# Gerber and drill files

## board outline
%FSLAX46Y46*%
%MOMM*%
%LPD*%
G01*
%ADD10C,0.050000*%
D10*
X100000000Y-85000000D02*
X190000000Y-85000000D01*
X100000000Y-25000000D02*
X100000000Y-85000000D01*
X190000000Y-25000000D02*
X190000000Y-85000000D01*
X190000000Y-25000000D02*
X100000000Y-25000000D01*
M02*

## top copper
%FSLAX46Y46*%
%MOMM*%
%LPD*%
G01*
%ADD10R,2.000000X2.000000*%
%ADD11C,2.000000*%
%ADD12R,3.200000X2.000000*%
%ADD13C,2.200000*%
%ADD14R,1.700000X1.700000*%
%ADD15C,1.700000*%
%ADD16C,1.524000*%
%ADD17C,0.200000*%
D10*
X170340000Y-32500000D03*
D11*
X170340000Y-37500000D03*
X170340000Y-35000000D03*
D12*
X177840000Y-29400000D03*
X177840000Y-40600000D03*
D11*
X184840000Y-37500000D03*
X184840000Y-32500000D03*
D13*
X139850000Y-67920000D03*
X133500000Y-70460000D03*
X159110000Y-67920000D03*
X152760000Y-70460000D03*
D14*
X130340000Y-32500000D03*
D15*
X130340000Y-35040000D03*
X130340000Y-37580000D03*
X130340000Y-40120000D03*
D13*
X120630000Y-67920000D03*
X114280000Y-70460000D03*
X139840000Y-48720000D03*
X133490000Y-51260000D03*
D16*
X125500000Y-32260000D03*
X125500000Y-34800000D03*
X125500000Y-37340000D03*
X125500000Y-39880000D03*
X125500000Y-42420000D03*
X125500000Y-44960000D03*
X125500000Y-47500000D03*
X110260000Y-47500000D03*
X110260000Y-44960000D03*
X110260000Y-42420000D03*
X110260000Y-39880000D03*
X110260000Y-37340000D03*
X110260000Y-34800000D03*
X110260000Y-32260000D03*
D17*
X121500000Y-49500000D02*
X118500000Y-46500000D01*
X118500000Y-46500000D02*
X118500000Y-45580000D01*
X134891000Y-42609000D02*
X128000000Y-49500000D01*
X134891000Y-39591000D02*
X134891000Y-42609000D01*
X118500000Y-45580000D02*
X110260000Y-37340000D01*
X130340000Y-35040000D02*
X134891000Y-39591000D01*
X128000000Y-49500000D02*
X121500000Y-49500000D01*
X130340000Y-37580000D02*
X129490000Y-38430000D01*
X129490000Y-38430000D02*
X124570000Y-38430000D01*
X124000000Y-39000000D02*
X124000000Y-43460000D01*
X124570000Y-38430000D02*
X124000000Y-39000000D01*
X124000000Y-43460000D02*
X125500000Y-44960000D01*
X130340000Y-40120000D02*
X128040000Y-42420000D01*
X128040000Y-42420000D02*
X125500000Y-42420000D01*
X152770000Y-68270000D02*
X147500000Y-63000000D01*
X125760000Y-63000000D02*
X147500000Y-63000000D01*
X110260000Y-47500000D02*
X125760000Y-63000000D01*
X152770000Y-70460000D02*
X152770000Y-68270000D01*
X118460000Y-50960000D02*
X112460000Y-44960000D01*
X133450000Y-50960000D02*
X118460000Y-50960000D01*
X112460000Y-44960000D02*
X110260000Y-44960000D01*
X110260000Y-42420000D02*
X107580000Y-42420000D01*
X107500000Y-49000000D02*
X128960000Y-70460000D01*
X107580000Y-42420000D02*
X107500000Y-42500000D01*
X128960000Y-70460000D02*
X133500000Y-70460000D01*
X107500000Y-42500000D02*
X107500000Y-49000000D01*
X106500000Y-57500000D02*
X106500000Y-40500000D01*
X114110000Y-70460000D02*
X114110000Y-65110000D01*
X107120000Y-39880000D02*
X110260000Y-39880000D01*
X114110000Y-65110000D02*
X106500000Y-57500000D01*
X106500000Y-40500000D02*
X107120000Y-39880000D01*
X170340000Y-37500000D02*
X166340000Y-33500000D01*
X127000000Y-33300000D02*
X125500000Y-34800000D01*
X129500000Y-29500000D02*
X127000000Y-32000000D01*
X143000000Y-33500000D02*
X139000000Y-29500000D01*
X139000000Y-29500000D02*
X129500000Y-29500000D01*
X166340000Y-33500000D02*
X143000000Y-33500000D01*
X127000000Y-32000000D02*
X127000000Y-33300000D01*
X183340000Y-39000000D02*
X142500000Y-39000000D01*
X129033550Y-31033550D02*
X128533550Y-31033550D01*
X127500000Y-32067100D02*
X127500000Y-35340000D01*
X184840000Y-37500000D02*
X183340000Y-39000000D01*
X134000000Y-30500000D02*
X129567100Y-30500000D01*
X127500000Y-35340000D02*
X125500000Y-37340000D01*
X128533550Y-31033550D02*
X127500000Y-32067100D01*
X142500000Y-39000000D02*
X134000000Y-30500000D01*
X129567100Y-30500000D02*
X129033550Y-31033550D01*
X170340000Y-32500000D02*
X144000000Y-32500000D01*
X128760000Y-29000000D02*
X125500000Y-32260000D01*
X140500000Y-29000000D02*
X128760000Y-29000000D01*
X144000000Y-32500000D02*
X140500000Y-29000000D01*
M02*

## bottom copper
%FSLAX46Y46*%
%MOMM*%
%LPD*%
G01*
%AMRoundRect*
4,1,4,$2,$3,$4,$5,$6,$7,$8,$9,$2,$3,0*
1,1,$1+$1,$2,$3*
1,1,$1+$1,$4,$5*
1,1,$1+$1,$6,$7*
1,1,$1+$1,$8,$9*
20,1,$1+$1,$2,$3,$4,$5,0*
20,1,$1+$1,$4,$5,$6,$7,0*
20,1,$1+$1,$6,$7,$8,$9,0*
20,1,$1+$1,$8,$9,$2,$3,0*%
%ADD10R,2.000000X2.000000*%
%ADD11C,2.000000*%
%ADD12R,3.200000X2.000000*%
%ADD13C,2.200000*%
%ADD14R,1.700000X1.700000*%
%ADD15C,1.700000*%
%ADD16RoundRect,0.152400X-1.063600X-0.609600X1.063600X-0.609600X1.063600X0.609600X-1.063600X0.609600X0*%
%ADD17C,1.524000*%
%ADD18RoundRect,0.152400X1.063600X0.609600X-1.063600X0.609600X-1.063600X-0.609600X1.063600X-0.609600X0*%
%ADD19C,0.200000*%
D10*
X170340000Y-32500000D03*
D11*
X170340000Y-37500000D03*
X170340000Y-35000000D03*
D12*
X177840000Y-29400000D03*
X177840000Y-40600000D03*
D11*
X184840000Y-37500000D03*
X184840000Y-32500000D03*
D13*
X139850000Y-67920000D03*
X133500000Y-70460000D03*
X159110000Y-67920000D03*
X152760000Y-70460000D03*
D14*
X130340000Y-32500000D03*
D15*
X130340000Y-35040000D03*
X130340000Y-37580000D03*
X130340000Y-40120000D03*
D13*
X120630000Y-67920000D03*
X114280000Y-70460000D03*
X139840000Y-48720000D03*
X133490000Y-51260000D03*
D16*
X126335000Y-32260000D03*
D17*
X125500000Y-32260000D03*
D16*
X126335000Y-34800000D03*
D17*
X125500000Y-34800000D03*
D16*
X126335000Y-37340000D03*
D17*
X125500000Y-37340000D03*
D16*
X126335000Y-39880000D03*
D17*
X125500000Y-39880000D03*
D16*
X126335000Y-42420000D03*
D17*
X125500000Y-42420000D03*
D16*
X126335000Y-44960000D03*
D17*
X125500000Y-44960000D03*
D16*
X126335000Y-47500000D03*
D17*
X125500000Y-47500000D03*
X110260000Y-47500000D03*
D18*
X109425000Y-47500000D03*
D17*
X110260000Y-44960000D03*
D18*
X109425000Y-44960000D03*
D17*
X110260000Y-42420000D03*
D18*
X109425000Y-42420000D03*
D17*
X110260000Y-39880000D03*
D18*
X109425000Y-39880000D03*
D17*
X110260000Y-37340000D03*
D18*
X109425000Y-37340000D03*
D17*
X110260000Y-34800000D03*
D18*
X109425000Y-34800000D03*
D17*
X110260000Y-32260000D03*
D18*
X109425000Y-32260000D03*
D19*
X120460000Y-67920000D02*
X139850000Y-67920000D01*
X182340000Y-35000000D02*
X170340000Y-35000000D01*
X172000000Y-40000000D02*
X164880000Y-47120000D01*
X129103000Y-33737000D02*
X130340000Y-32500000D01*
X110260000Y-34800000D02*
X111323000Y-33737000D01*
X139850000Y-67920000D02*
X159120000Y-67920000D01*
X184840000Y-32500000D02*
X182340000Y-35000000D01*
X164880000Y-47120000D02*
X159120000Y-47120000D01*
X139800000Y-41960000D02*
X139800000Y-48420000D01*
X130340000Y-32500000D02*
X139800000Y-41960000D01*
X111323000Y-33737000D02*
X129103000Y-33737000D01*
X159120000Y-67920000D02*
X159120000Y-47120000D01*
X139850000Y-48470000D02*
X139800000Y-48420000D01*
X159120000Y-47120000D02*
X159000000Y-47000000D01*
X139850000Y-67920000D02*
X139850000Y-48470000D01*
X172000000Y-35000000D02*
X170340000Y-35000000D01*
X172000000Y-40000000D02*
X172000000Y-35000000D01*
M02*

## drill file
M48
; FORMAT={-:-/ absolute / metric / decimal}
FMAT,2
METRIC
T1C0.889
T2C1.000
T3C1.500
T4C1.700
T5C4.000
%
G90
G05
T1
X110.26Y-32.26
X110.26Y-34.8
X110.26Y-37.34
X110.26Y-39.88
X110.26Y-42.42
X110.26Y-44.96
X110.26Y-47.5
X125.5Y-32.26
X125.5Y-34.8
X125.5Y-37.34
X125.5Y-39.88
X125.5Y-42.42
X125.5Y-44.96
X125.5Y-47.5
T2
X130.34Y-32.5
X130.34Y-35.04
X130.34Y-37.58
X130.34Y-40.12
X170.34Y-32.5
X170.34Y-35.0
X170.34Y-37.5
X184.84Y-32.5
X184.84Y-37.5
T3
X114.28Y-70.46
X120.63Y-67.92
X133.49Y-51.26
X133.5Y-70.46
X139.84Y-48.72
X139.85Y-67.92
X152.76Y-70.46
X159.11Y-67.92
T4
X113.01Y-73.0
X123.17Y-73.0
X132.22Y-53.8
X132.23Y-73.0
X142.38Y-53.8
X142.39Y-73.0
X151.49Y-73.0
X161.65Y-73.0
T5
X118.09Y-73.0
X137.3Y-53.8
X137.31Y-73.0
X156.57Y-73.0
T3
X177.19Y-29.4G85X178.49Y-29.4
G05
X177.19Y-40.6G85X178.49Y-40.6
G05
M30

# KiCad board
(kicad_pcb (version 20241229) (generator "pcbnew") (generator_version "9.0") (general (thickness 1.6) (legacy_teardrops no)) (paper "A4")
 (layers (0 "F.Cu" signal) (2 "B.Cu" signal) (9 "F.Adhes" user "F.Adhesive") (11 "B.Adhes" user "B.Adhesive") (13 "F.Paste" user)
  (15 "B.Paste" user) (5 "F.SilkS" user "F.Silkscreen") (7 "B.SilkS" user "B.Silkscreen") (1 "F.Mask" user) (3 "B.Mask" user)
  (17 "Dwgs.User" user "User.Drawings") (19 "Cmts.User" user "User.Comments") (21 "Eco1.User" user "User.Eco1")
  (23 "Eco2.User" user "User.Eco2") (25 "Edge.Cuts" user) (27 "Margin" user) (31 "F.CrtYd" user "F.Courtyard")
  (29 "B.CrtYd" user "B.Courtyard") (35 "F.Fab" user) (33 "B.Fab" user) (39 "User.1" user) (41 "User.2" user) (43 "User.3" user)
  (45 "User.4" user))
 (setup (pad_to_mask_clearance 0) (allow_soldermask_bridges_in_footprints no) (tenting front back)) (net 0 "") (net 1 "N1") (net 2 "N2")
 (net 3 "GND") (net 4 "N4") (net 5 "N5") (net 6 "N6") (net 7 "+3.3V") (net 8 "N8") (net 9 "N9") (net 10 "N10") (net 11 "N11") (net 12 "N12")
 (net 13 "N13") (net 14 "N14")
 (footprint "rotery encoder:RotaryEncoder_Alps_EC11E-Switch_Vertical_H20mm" (layer "F.Cu") (at 170.34 32.5)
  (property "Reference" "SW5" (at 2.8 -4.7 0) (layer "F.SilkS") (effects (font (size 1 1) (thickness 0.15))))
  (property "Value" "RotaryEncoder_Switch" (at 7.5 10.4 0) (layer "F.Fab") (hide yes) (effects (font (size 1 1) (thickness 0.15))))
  (pad "A" thru_hole rect (at 0 0) (size 2 2) (drill 1) (layers "*.Cu" "*.Mask") (remove_unused_layers no) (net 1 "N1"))
  (pad "B" thru_hole circle (at 0 5) (size 2 2) (drill 1) (layers "*.Cu" "*.Mask") (remove_unused_layers no) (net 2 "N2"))
  (pad "C" thru_hole circle (at 0 2.5) (size 2 2) (drill 1) (layers "*.Cu" "*.Mask") (remove_unused_layers no) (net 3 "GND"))
  (pad "MP" thru_hole rect (at 7.5 -3.1) (size 3.2 2) (drill oval 2.8 1.5) (layers "*.Cu" "*.Mask") (remove_unused_layers no))
  (pad "MP" thru_hole rect (at 7.5 8.1) (size 3.2 2) (drill oval 2.8 1.5) (layers "*.Cu" "*.Mask") (remove_unused_layers no))
  (pad "S1" thru_hole circle (at 14.5 5) (size 2 2) (drill 1) (layers "*.Cu" "*.Mask") (remove_unused_layers no) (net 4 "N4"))
  (pad "S2" thru_hole circle (at 14.5 0) (size 2 2) (drill 1) (layers "*.Cu" "*.Mask") (remove_unused_layers no) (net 3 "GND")))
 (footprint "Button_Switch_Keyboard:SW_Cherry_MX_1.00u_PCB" (layer "F.Cu") (at 139.85 67.92)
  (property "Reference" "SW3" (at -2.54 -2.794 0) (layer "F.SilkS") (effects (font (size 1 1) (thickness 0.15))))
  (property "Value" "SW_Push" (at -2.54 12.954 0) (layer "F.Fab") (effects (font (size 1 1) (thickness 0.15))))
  (pad "" np_thru_hole circle (at -7.62 5.08) (size 1.7 1.7) (drill 1.7) (layers "*.Cu" "*.Mask"))
  (pad "" np_thru_hole circle (at -2.54 5.08) (size 4 4) (drill 4) (layers "*.Cu" "*.Mask"))
  (pad "" np_thru_hole circle (at 2.54 5.08) (size 1.7 1.7) (drill 1.7) (layers "*.Cu" "*.Mask"))
  (pad "1" thru_hole circle (at 0 0) (size 2.2 2.2) (drill 1.5) (layers "*.Cu" "*.Mask") (remove_unused_layers no) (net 3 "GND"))
  (pad "2" thru_hole circle (at -6.35 2.54) (size 2.2 2.2) (drill 1.5) (layers "*.Cu" "*.Mask") (remove_unused_layers no) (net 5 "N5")))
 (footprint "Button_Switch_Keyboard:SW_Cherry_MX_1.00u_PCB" (layer "F.Cu") (at 159.11 67.92)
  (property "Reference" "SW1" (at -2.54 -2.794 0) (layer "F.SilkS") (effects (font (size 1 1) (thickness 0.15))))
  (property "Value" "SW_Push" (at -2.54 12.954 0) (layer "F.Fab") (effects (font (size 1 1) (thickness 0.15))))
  (pad "" np_thru_hole circle (at -7.62 5.08) (size 1.7 1.7) (drill 1.7) (layers "*.Cu" "*.Mask"))
  (pad "" np_thru_hole circle (at -2.54 5.08) (size 4 4) (drill 4) (layers "*.Cu" "*.Mask"))
  (pad "" np_thru_hole circle (at 2.54 5.08) (size 1.7 1.7) (drill 1.7) (layers "*.Cu" "*.Mask"))
  (pad "1" thru_hole circle (at 0 0) (size 2.2 2.2) (drill 1.5) (layers "*.Cu" "*.Mask") (remove_unused_layers no) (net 3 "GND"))
  (pad "2" thru_hole circle (at -6.35 2.54) (size 2.2 2.2) (drill 1.5) (layers "*.Cu" "*.Mask") (remove_unused_layers no) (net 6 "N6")))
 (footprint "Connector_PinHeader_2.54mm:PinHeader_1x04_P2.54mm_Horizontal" (layer "F.Cu") (at 130.34 32.5)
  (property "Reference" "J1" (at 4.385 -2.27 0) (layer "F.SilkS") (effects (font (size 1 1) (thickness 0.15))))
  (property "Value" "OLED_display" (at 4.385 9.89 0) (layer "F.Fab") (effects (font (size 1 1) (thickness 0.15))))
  (pad "1" thru_hole rect (at 0 0) (size 1.7 1.7) (drill 1) (layers "*.Cu" "*.Mask") (remove_unused_layers no) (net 3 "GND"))
  (pad "2" thru_hole circle (at 0 2.54) (size 1.7 1.7) (drill 1) (layers "*.Cu" "*.Mask") (remove_unused_layers no) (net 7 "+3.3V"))
  (pad "3" thru_hole circle (at 0 5.08) (size 1.7 1.7) (drill 1) (layers "*.Cu" "*.Mask") (remove_unused_layers no) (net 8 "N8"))
  (pad "4" thru_hole circle (at 0 7.62) (size 1.7 1.7) (drill 1) (layers "*.Cu" "*.Mask") (remove_unused_layers no) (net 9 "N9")))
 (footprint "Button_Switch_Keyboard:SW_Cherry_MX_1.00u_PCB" (layer "F.Cu") (at 120.63 67.92)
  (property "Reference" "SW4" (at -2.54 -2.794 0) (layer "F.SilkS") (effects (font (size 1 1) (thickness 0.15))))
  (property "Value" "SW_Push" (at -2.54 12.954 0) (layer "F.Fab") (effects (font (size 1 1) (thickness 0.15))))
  (pad "" np_thru_hole circle (at -7.62 5.08) (size 1.7 1.7) (drill 1.7) (layers "*.Cu" "*.Mask"))
  (pad "" np_thru_hole circle (at -2.54 5.08) (size 4 4) (drill 4) (layers "*.Cu" "*.Mask"))
  (pad "" np_thru_hole circle (at 2.54 5.08) (size 1.7 1.7) (drill 1.7) (layers "*.Cu" "*.Mask"))
  (pad "1" thru_hole circle (at 0 0) (size 2.2 2.2) (drill 1.5) (layers "*.Cu" "*.Mask") (remove_unused_layers no) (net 3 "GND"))
  (pad "2" thru_hole circle (at -6.35 2.54) (size 2.2 2.2) (drill 1.5) (layers "*.Cu" "*.Mask") (remove_unused_layers no) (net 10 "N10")))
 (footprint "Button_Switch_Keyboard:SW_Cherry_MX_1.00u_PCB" (layer "F.Cu") (at 139.84 48.72)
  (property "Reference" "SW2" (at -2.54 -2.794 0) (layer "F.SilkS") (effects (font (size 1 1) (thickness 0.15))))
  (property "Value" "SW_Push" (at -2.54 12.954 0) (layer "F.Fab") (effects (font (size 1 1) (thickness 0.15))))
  (pad "" np_thru_hole circle (at -7.62 5.08) (size 1.7 1.7) (drill 1.7) (layers "*.Cu" "*.Mask"))
  (pad "" np_thru_hole circle (at -2.54 5.08) (size 4 4) (drill 4) (layers "*.Cu" "*.Mask"))
  (pad "" np_thru_hole circle (at 2.54 5.08) (size 1.7 1.7) (drill 1.7) (layers "*.Cu" "*.Mask"))
  (pad "1" thru_hole circle (at 0 0) (size 2.2 2.2) (drill 1.5) (layers "*.Cu" "*.Mask") (remove_unused_layers no) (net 3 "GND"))
  (pad "2" thru_hole circle (at -6.35 2.54) (size 2.2 2.2) (drill 1.5) (layers "*.Cu" "*.Mask") (remove_unused_layers no) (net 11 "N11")))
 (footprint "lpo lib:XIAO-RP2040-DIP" (layer "B.Cu") (at 117.88 39.88 180)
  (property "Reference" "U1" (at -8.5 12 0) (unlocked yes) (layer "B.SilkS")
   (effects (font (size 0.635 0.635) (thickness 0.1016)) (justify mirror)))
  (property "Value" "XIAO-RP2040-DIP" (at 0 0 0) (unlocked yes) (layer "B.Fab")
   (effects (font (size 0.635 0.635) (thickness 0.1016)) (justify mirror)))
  (pad "1" smd roundrect (at -8.455 7.62) (size 2.432 1.524) (layers "B.Cu" "B.Mask") (roundrect_rratio 0.1) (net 1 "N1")
   (thermal_bridge_angle 45))
  (pad "1" thru_hole circle (at -7.62 7.62) (size 1.524 1.524) (drill 0.889) (layers "*.Cu" "*.Mask") (remove_unused_layers no) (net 1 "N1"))
  (pad "2" smd roundrect (at -8.455 5.08) (size 2.432 1.524) (layers "B.Cu" "B.Mask") (roundrect_rratio 0.1) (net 2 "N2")
   (thermal_bridge_angle 45))
  (pad "2" thru_hole circle (at -7.62 5.08) (size 1.524 1.524) (drill 0.889) (layers "*.Cu" "*.Mask") (remove_unused_layers no) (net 2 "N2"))
  (pad "3" smd roundrect (at -8.455 2.54) (size 2.432 1.524) (layers "B.Cu" "B.Mask") (roundrect_rratio 0.1) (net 4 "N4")
   (thermal_bridge_angle 45))
  (pad "3" thru_hole circle (at -7.62 2.54) (size 1.524 1.524) (drill 0.889) (layers "*.Cu" "*.Mask") (remove_unused_layers no) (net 4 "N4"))
  (pad "4" smd roundrect (at -8.455 0) (size 2.432 1.524) (layers "B.Cu" "B.Mask") (roundrect_rratio 0.1) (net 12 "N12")
   (thermal_bridge_angle 45))
  (pad "4" thru_hole circle (at -7.62 0) (size 1.524 1.524) (drill 0.889) (layers "*.Cu" "*.Mask") (remove_unused_layers no) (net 12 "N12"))
  (pad "5" smd roundrect (at -8.455 -2.54) (size 2.432 1.524) (layers "B.Cu" "B.Mask") (roundrect_rratio 0.1) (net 9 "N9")
   (thermal_bridge_angle 45))
  (pad "5" thru_hole circle (at -7.62 -2.54) (size 1.524 1.524) (drill 0.889) (layers "*.Cu" "*.Mask") (remove_unused_layers no)
   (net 9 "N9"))
  (pad "6" smd roundrect (at -8.455 -5.08) (size 2.432 1.524) (layers "B.Cu" "B.Mask") (roundrect_rratio 0.1) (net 8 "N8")
   (thermal_bridge_angle 45))
  (pad "6" thru_hole circle (at -7.62 -5.08) (size 1.524 1.524) (drill 0.889) (layers "*.Cu" "*.Mask") (remove_unused_layers no)
   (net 8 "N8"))
  (pad "7" smd roundrect (at -8.455 -7.62) (size 2.432 1.524) (layers "B.Cu" "B.Mask") (roundrect_rratio 0.1) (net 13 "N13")
   (thermal_bridge_angle 45))
  (pad "7" thru_hole circle (at -7.62 -7.62) (size 1.524 1.524) (drill 0.889) (layers "*.Cu" "*.Mask") (remove_unused_layers no)
   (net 13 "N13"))
  (pad "8" thru_hole circle (at 7.62 -7.62 180) (size 1.524 1.524) (drill 0.889) (layers "*.Cu" "*.Mask") (remove_unused_layers no)
   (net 6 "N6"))
  (pad "8" smd roundrect (at 8.455 -7.62 180) (size 2.432 1.524) (layers "B.Cu" "B.Mask") (roundrect_rratio 0.1) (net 6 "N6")
   (thermal_bridge_angle 45))
  (pad "9" thru_hole circle (at 7.62 -5.08 180) (size 1.524 1.524) (drill 0.889) (layers "*.Cu" "*.Mask") (remove_unused_layers no)
   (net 11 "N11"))
  (pad "9" smd roundrect (at 8.455 -5.08 180) (size 2.432 1.524) (layers "B.Cu" "B.Mask") (roundrect_rratio 0.1) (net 11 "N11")
   (thermal_bridge_angle 45))
  (pad "10" thru_hole circle (at 7.62 -2.54 180) (size 1.524 1.524) (drill 0.889) (layers "*.Cu" "*.Mask") (remove_unused_layers no)
   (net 5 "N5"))
  (pad "10" smd roundrect (at 8.455 -2.54 180) (size 2.432 1.524) (layers "B.Cu" "B.Mask") (roundrect_rratio 0.1) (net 5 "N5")
   (thermal_bridge_angle 45))
  (pad "11" thru_hole circle (at 7.62 0 180) (size 1.524 1.524) (drill 0.889) (layers "*.Cu" "*.Mask") (remove_unused_layers no)
   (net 10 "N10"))
  (pad "11" smd roundrect (at 8.455 0 180) (size 2.432 1.524) (layers "B.Cu" "B.Mask") (roundrect_rratio 0.1) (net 10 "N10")
   (thermal_bridge_angle 45))
  (pad "12" thru_hole circle (at 7.62 2.54 180) (size 1.524 1.524) (drill 0.889) (layers "*.Cu" "*.Mask") (remove_unused_layers no)
   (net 7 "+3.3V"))
  (pad "12" smd roundrect (at 8.455 2.54 180) (size 2.432 1.524) (layers "B.Cu" "B.Mask") (roundrect_rratio 0.1) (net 7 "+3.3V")
   (thermal_bridge_angle 45))
  (pad "13" thru_hole circle (at 7.62 5.08 180) (size 1.524 1.524) (drill 0.889) (layers "*.Cu" "*.Mask") (remove_unused_layers no)
   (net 3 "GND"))
  (pad "13" smd roundrect (at 8.455 5.08 180) (size 2.432 1.524) (layers "B.Cu" "B.Mask") (roundrect_rratio 0.1) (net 3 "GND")
   (thermal_bridge_angle 45))
  (pad "14" thru_hole circle (at 7.62 7.62 180) (size 1.524 1.524) (drill 0.889) (layers "*.Cu" "*.Mask") (remove_unused_layers no)
   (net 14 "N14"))
  (pad "14" smd roundrect (at 8.455 7.62 180) (size 2.432 1.524) (layers "B.Cu" "B.Mask") (roundrect_rratio 0.1) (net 14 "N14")
   (thermal_bridge_angle 45)))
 (gr_line (start 100 85) (end 190 85) (stroke (width 0.05) (type default)) (layer "Edge.Cuts"))
 (gr_line (start 100 25) (end 100 85) (stroke (width 0.05) (type default)) (layer "Edge.Cuts"))
 (gr_line (start 190 25) (end 190 85) (stroke (width 0.05) (type default)) (layer "Edge.Cuts"))
 (gr_line (start 190 25) (end 100 25) (stroke (width 0.05) (type default)) (layer "Edge.Cuts"))
 (segment (start 121.5 49.5) (end 118.5 46.5) (width 0.2) (layer "F.Cu") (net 7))
 (segment (start 118.5 46.5) (end 118.5 45.58) (width 0.2) (layer "F.Cu") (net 7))
 (segment (start 134.891 42.609) (end 128 49.5) (width 0.2) (layer "F.Cu") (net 7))
 (segment (start 134.891 39.591) (end 134.891 42.609) (width 0.2) (layer "F.Cu") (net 7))
 (segment (start 118.5 45.58) (end 110.26 37.34) (width 0.2) (layer "F.Cu") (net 7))
 (segment (start 130.34 35.04) (end 134.891 39.591) (width 0.2) (layer "F.Cu") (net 7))
 (segment (start 128 49.5) (end 121.5 49.5) (width 0.2) (layer "F.Cu") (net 7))
 (segment (start 120.46 67.92) (end 139.85 67.92) (width 0.2) (layer "B.Cu") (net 3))
 (segment (start 182.34 35) (end 170.34 35) (width 0.2) (layer "B.Cu") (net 3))
 (segment (start 172 40) (end 164.88 47.12) (width 0.2) (layer "B.Cu") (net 3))
 (segment (start 129.103 33.737) (end 130.34 32.5) (width 0.2) (layer "B.Cu") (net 3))
 (segment (start 110.26 34.8) (end 111.323 33.737) (width 0.2) (layer "B.Cu") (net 3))
 (segment (start 139.85 67.92) (end 159.12 67.92) (width 0.2) (layer "B.Cu") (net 3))
 (segment (start 184.84 32.5) (end 182.34 35) (width 0.2) (layer "B.Cu") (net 3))
 (segment (start 164.88 47.12) (end 159.12 47.12) (width 0.2) (layer "B.Cu") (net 3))
 (segment (start 139.8 41.96) (end 139.8 48.42) (width 0.2) (layer "B.Cu") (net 3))
 (segment (start 130.34 32.5) (end 139.8 41.96) (width 0.2) (layer "B.Cu") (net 3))
 (segment (start 111.323 33.737) (end 129.103 33.737) (width 0.2) (layer "B.Cu") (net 3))
 (segment (start 159.12 67.92) (end 159.12 47.12) (width 0.2) (layer "B.Cu") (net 3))
 (segment (start 139.85 48.47) (end 139.8 48.42) (width 0.2) (layer "B.Cu") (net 3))
 (segment (start 159.12 47.12) (end 159 47) (width 0.2) (layer "B.Cu") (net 3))
 (segment (start 139.85 67.92) (end 139.85 48.47) (width 0.2) (layer "B.Cu") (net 3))
 (segment (start 172 35) (end 170.34 35) (width 0.2) (layer "B.Cu") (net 3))
 (segment (start 172 40) (end 172 35) (width 0.2) (layer "B.Cu") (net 3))
 (segment (start 130.34 37.58) (end 129.49 38.43) (width 0.2) (layer "F.Cu") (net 8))
 (segment (start 129.49 38.43) (end 124.57 38.43) (width 0.2) (layer "F.Cu") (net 8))
 (segment (start 124 39) (end 124 43.46) (width 0.2) (layer "F.Cu") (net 8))
 (segment (start 124.57 38.43) (end 124 39) (width 0.2) (layer "F.Cu") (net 8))
 (segment (start 124 43.46) (end 125.5 44.96) (width 0.2) (layer "F.Cu") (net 8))
 (segment (start 130.34 40.12) (end 128.04 42.42) (width 0.2) (layer "F.Cu") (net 9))
 (segment (start 128.04 42.42) (end 125.5 42.42) (width 0.2) (layer "F.Cu") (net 9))
 (segment (start 152.77 68.27) (end 147.5 63) (width 0.2) (layer "F.Cu") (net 6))
 (segment (start 125.76 63) (end 147.5 63) (width 0.2) (layer "F.Cu") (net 6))
 (segment (start 110.26 47.5) (end 125.76 63) (width 0.2) (layer "F.Cu") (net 6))
 (segment (start 152.77 70.46) (end 152.77 68.27) (width 0.2) (layer "F.Cu") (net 6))
 (segment (start 118.46 50.96) (end 112.46 44.96) (width 0.2) (layer "F.Cu") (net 11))
 (segment (start 133.45 50.96) (end 118.46 50.96) (width 0.2) (layer "F.Cu") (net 11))
 (segment (start 112.46 44.96) (end 110.26 44.96) (width 0.2) (layer "F.Cu") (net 11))
 (segment (start 110.26 42.42) (end 107.58 42.42) (width 0.2) (layer "F.Cu") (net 5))
 (segment (start 107.5 49) (end 128.96 70.46) (width 0.2) (layer "F.Cu") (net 5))
 (segment (start 107.58 42.42) (end 107.5 42.5) (width 0.2) (layer "F.Cu") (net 5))
 (segment (start 128.96 70.46) (end 133.5 70.46) (width 0.2) (layer "F.Cu") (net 5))
 (segment (start 107.5 42.5) (end 107.5 49) (width 0.2) (layer "F.Cu") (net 5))
 (segment (start 106.5 57.5) (end 106.5 40.5) (width 0.2) (layer "F.Cu") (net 10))
 (segment (start 114.11 70.46) (end 114.11 65.11) (width 0.2) (layer "F.Cu") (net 10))
 (segment (start 107.12 39.88) (end 110.26 39.88) (width 0.2) (layer "F.Cu") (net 10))
 (segment (start 114.11 65.11) (end 106.5 57.5) (width 0.2) (layer "F.Cu") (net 10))
 (segment (start 106.5 40.5) (end 107.12 39.88) (width 0.2) (layer "F.Cu") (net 10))
 (segment (start 170.34 37.5) (end 166.34 33.5) (width 0.2) (layer "F.Cu") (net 2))
 (segment (start 127 33.3) (end 125.5 34.8) (width 0.2) (layer "F.Cu") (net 2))
 (segment (start 129.5 29.5) (end 127 32) (width 0.2) (layer "F.Cu") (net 2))
 (segment (start 143 33.5) (end 139 29.5) (width 0.2) (layer "F.Cu") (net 2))
 (segment (start 139 29.5) (end 129.5 29.5) (width 0.2) (layer "F.Cu") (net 2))
 (segment (start 166.34 33.5) (end 143 33.5) (width 0.2) (layer "F.Cu") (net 2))
 (segment (start 127 32) (end 127 33.3) (width 0.2) (layer "F.Cu") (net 2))
 (segment (start 183.34 39) (end 142.5 39) (width 0.2) (layer "F.Cu") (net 4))
 (segment (start 129.03355 31.03355) (end 128.53355 31.03355) (width 0.2) (layer "F.Cu") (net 4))
 (segment (start 127.5 32.0671) (end 127.5 35.34) (width 0.2) (layer "F.Cu") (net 4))
 (segment (start 184.84 37.5) (end 183.34 39) (width 0.2) (layer "F.Cu") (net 4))
 (segment (start 134 30.5) (end 129.5671 30.5) (width 0.2) (layer "F.Cu") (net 4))
 (segment (start 127.5 35.34) (end 125.5 37.34) (width 0.2) (layer "F.Cu") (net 4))
 (segment (start 128.53355 31.03355) (end 127.5 32.0671) (width 0.2) (layer "F.Cu") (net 4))
 (segment (start 142.5 39) (end 134 30.5) (width 0.2) (layer "F.Cu") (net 4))
 (segment (start 129.5671 30.5) (end 129.03355 31.03355) (width 0.2) (layer "F.Cu") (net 4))
 (segment (start 170.34 32.5) (end 144 32.5) (width 0.2) (layer "F.Cu") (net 1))
 (segment (start 128.76 29) (end 125.5 32.26) (width 0.2) (layer "F.Cu") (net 1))
 (segment (start 140.5 29) (end 128.76 29) (width 0.2) (layer "F.Cu") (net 1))
 (segment (start 144 32.5) (end 140.5 29) (width 0.2) (layer "F.Cu") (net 1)))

